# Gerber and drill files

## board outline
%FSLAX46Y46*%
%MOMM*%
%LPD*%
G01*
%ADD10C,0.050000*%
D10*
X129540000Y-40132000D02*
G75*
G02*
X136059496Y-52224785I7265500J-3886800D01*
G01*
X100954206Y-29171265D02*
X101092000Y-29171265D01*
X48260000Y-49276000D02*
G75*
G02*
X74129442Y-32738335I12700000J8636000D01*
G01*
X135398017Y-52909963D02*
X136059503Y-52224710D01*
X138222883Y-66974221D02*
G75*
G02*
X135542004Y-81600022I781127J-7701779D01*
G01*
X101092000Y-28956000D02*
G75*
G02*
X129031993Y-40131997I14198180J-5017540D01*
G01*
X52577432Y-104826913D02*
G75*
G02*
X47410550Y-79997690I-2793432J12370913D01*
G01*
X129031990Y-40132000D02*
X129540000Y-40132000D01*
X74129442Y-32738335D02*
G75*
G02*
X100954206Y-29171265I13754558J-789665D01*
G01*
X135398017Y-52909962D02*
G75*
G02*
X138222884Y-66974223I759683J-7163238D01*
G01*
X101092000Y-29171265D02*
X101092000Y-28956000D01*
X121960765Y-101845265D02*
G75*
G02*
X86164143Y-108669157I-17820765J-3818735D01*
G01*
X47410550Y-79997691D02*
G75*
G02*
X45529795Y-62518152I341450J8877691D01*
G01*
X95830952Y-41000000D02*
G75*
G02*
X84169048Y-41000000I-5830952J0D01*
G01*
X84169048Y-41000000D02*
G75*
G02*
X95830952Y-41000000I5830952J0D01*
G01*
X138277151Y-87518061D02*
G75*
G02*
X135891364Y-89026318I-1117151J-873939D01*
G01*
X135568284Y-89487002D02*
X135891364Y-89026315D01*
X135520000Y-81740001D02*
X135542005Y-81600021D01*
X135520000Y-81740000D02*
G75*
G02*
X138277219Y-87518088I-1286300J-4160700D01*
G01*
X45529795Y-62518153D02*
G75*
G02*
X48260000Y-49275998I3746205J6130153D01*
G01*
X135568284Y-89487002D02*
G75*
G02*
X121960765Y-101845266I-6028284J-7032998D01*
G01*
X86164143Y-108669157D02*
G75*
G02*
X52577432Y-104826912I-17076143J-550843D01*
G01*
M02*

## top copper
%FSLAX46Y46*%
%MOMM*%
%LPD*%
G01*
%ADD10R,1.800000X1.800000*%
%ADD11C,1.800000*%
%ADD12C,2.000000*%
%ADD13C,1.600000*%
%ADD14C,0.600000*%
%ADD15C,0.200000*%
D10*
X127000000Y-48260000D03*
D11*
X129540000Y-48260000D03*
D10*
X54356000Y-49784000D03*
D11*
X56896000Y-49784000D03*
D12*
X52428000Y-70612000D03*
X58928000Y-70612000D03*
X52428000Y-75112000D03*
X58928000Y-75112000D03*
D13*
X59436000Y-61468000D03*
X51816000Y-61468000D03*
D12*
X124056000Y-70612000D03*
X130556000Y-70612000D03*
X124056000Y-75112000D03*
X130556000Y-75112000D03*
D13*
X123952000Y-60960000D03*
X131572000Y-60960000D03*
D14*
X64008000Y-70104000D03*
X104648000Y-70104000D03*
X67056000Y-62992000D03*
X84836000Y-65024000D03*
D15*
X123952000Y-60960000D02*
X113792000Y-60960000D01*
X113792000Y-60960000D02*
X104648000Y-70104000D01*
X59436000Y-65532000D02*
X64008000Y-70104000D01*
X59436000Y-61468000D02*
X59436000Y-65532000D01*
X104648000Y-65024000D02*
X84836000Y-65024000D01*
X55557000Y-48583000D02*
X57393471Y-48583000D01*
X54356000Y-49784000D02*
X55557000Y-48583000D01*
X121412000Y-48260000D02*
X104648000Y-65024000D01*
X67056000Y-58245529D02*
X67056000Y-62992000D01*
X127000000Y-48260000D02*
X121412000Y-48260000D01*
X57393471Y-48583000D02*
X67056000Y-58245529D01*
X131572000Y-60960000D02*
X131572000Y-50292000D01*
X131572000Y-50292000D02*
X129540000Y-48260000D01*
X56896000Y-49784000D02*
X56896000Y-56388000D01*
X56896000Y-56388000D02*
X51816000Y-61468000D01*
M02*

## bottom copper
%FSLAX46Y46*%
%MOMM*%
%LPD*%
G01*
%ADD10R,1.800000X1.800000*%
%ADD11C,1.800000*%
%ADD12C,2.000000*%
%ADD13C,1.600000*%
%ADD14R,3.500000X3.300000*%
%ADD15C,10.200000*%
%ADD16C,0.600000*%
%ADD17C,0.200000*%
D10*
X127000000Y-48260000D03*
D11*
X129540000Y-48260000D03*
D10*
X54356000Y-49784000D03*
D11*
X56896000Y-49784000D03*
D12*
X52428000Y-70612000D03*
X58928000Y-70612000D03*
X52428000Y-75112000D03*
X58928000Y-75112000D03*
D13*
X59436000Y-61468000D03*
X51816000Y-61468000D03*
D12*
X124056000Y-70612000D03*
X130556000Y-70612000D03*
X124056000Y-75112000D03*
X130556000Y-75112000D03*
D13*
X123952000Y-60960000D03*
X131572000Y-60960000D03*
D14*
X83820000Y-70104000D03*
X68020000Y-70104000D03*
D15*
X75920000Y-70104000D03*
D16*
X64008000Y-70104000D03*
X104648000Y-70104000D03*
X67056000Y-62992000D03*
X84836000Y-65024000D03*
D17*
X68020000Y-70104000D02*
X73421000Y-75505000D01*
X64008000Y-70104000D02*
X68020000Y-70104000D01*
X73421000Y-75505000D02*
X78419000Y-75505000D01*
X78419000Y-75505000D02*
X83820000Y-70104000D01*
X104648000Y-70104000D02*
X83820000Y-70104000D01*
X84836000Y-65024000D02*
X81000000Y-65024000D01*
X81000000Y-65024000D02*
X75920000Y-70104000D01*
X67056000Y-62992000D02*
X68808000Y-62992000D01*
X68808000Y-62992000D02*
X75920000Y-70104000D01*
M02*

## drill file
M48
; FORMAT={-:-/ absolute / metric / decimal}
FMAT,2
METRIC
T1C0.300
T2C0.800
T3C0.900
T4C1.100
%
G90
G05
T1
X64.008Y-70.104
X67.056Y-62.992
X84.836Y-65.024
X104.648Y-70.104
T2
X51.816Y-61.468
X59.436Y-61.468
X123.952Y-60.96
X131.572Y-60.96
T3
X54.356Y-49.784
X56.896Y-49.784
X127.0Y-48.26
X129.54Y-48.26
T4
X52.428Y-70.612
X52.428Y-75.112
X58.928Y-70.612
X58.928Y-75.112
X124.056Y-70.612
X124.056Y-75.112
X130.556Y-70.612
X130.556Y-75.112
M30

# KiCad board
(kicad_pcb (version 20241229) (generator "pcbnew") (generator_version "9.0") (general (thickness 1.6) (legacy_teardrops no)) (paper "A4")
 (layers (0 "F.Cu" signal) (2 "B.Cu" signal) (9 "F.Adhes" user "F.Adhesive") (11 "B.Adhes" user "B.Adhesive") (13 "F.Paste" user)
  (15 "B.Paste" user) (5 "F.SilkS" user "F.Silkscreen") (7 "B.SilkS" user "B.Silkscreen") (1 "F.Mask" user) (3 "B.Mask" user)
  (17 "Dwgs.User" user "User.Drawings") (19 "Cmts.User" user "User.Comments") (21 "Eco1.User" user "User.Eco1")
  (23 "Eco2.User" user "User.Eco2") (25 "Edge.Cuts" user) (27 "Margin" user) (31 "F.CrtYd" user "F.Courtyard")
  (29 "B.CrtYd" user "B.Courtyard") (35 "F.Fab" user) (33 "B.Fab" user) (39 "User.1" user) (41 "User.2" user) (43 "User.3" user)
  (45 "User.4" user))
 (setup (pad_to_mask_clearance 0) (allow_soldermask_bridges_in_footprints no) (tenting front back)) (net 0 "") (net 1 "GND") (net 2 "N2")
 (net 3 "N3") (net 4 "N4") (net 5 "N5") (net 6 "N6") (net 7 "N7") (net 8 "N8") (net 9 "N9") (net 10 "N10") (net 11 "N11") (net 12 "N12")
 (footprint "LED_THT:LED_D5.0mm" (layer "F.Cu") (at 127 48.26)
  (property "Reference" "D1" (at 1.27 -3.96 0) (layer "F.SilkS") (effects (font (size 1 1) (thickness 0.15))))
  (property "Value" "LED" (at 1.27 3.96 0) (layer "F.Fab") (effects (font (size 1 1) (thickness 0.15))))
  (pad "1" thru_hole rect (at 0 0) (size 1.8 1.8) (drill 0.9) (layers "*.Cu" "*.Mask") (remove_unused_layers no) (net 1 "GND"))
  (pad "2" thru_hole circle (at 2.54 0) (size 1.8 1.8) (drill 0.9) (layers "*.Cu" "*.Mask") (remove_unused_layers no) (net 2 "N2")))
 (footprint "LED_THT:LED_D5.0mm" (layer "F.Cu") (at 54.356 49.784)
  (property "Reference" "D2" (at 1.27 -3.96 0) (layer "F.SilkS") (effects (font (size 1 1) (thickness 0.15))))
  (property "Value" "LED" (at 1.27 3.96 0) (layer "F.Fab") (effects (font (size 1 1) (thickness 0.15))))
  (pad "1" thru_hole rect (at 0 0) (size 1.8 1.8) (drill 0.9) (layers "*.Cu" "*.Mask") (remove_unused_layers no) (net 1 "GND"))
  (pad "2" thru_hole circle (at 2.54 0) (size 1.8 1.8) (drill 0.9) (layers "*.Cu" "*.Mask") (remove_unused_layers no) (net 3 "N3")))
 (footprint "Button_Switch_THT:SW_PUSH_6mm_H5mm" (layer "F.Cu") (at 52.428 70.612)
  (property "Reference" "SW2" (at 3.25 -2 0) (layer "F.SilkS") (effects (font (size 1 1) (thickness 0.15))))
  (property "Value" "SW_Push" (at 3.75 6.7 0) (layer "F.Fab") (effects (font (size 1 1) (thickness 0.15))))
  (pad "1" thru_hole circle (at 0 0 90) (size 2 2) (drill 1.1) (layers "*.Cu" "*.Mask") (remove_unused_layers no) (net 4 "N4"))
  (pad "1" thru_hole circle (at 6.5 0 90) (size 2 2) (drill 1.1) (layers "*.Cu" "*.Mask") (remove_unused_layers no) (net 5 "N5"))
  (pad "2" thru_hole circle (at 0 4.5 90) (size 2 2) (drill 1.1) (layers "*.Cu" "*.Mask") (remove_unused_layers no) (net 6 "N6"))
  (pad "2" thru_hole circle (at 6.5 4.5 90) (size 2 2) (drill 1.1) (layers "*.Cu" "*.Mask") (remove_unused_layers no) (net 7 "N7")))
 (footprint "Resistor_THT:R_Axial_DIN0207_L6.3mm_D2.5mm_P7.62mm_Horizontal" (layer "F.Cu") (at 59.436 61.468 180)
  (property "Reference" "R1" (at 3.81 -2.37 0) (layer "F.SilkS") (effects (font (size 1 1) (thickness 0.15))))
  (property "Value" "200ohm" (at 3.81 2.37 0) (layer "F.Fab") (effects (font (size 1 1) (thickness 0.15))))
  (pad "1" thru_hole circle (at 0 0 180) (size 1.6 1.6) (drill 0.8) (layers "*.Cu" "*.Mask") (remove_unused_layers no) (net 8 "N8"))
  (pad "2" thru_hole circle (at 7.62 0 180) (size 1.6 1.6) (drill 0.8) (layers "*.Cu" "*.Mask") (remove_unused_layers no) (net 3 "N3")))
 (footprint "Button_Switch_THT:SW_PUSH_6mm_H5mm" (layer "F.Cu") (at 124.056 70.612)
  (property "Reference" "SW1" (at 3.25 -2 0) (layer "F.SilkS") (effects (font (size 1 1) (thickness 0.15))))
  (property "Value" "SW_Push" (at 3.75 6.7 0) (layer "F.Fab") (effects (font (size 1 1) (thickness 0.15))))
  (pad "1" thru_hole circle (at 0 0 90) (size 2 2) (drill 1.1) (layers "*.Cu" "*.Mask") (remove_unused_layers no) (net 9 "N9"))
  (pad "1" thru_hole circle (at 6.5 0 90) (size 2 2) (drill 1.1) (layers "*.Cu" "*.Mask") (remove_unused_layers no) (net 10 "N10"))
  (pad "2" thru_hole circle (at 0 4.5 90) (size 2 2) (drill 1.1) (layers "*.Cu" "*.Mask") (remove_unused_layers no) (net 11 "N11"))
  (pad "2" thru_hole circle (at 6.5 4.5 90) (size 2 2) (drill 1.1) (layers "*.Cu" "*.Mask") (remove_unused_layers no) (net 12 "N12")))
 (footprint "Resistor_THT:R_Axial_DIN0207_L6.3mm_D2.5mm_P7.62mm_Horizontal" (layer "F.Cu") (at 123.952 60.96)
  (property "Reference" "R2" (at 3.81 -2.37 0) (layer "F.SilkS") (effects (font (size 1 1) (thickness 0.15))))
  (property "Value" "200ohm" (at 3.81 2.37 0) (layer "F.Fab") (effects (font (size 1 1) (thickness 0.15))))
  (pad "1" thru_hole circle (at 0 0) (size 1.6 1.6) (drill 0.8) (layers "*.Cu" "*.Mask") (remove_unused_layers no) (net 8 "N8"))
  (pad "2" thru_hole circle (at 7.62 0) (size 1.6 1.6) (drill 0.8) (layers "*.Cu" "*.Mask") (remove_unused_layers no) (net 2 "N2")))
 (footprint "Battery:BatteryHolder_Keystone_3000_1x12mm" (layer "B.Cu") (at 75.92 70.104 180)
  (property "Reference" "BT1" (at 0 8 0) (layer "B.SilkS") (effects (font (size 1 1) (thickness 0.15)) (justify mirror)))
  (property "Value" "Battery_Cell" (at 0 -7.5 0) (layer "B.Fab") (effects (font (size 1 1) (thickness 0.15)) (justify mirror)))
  (pad "1" smd rect (at -7.9 0 180) (size 3.5 3.3) (layers "B.Cu" "B.Mask" "B.Paste") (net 8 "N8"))
  (pad "1" smd rect (at 7.9 0 180) (size 3.5 3.3) (layers "B.Cu" "B.Mask" "B.Paste") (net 8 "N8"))
  (pad "2" smd circle (at 0 0 180) (size 10.2 10.2) (layers "B.Cu" "B.Mask") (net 1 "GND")))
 (gr_arc (start 129.54 40.132) (mid 144.058392 40.108523) (end 136.059503 52.224712) (stroke (width 0.05) (type default))
  (layer "Edge.Cuts"))
 (gr_line (start 100.954206 29.171265) (end 101.092 29.171265) (stroke (width 0.05) (type default)) (layer "Edge.Cuts"))
 (gr_arc (start 48.26 49.276) (mid 52.687837 27.700069) (end 74.129442 32.738335) (stroke (width 0.05) (type default)) (layer "Edge.Cuts"))
 (gr_line (start 135.398017 52.909963) (end 136.059503 52.22471) (stroke (width 0.05) (type default)) (layer "Edge.Cuts"))
 (gr_arc (start 138.222883 66.974221) (mid 146.618446 76.071709) (end 135.542005 81.60002) (stroke (width 0.05) (type default))
  (layer "Edge.Cuts"))
 (gr_arc (start 101.092 28.956) (mid 120.882838 19.991901) (end 129.032 40.132) (stroke (width 0.05) (type default)) (layer "Edge.Cuts"))
 (gr_arc (start 52.577432 104.826913) (mid 37.367613 95.039811) (end 47.41055 79.99769) (stroke (width 0.05) (type default))
  (layer "Edge.Cuts"))
 (gr_line (start 129.03199 40.132) (end 129.54 40.132) (stroke (width 0.05) (type default)) (layer "Edge.Cuts"))
 (gr_arc (start 74.129442 32.738335) (mid 86.067938 19.871011) (end 100.954206 29.171265) (stroke (width 0.05) (type default))
  (layer "Edge.Cuts"))
 (gr_arc (start 135.398017 52.909962) (mid 143.220055 58.654695) (end 138.222883 66.974221) (stroke (width 0.05) (type default))
  (layer "Edge.Cuts"))
 (gr_line (start 101.092 29.171265) (end 101.092 28.956) (stroke (width 0.05) (type default)) (layer "Edge.Cuts"))
 (gr_arc (start 121.960765 101.845265) (mid 107.552827 123.566933) (end 86.164143 108.669157) (stroke (width 0.05) (type default))
  (layer "Edge.Cuts"))
 (gr_arc (start 47.41055 79.997691) (mid 38.91873 72.070438) (end 45.529795 62.518152) (stroke (width 0.05) (type default))
  (layer "Edge.Cuts"))
 (gr_circle (center 90 41) (end 85 38) (stroke (width 0.05) (type default)) (fill no) (layer "Edge.Cuts"))
 (gr_arc (start 138.277151 87.518061) (mid 137.917923 89.590895) (end 135.891364 89.026318) (stroke (width 0.05) (type default))
  (layer "Edge.Cuts"))
 (gr_line (start 135.568284 89.487002) (end 135.891364 89.026315) (stroke (width 0.05) (type default)) (layer "Edge.Cuts"))
 (gr_line (start 135.52 81.740001) (end 135.542005 81.600021) (stroke (width 0.05) (type default)) (layer "Edge.Cuts"))
 (gr_arc (start 135.52 81.74) (mid 138.164098 84.025154) (end 138.277153 87.518061) (stroke (width 0.05) (type default)) (layer "Edge.Cuts"))
 (gr_arc (start 45.529795 62.518153) (mid 42.239785 54.937306) (end 48.26 49.275998) (stroke (width 0.05) (type default))
  (layer "Edge.Cuts"))
 (gr_arc (start 135.568284 89.487002) (mid 135.767603 103.37713) (end 121.960765 101.845266) (stroke (width 0.05) (type default))
  (layer "Edge.Cuts"))
 (gr_arc (start 86.164143 108.669157) (mid 67.146176 126.194316) (end 52.577432 104.826912) (stroke (width 0.05) (type default))
  (layer "Edge.Cuts"))
 (segment (start 123.952 60.96) (end 113.792 60.96) (width 0.2) (layer "F.Cu") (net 8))
 (segment (start 113.792 60.96) (end 104.648 70.104) (width 0.2) (layer "F.Cu") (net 8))
 (segment (start 59.436 65.532) (end 64.008 70.104) (width 0.2) (layer "F.Cu") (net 8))
 (segment (start 59.436 61.468) (end 59.436 65.532) (width 0.2) (layer "F.Cu") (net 8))
 (via (at 64.008 70.104) (size 0.6) (drill 0.3) (layers "F.Cu" "B.Cu") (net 8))
 (via (at 104.648 70.104) (size 0.6) (drill 0.3) (layers "F.Cu" "B.Cu") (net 8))
 (segment (start 68.02 70.104) (end 73.421 75.505) (width 0.2) (layer "B.Cu") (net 8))
 (segment (start 64.008 70.104) (end 68.02 70.104) (width 0.2) (layer "B.Cu") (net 8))
 (segment (start 73.421 75.505) (end 78.419 75.505) (width 0.2) (layer "B.Cu") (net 8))
 (segment (start 78.419 75.505) (end 83.82 70.104) (width 0.2) (layer "B.Cu") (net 8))
 (segment (start 104.648 70.104) (end 83.82 70.104) (width 0.2) (layer "B.Cu") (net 8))
 (segment (start 104.648 65.024) (end 84.836 65.024) (width 0.2) (layer "F.Cu") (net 1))
 (segment (start 55.557 48.583) (end 57.393471 48.583) (width 0.2) (layer "F.Cu") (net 1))
 (segment (start 54.356 49.784) (end 55.557 48.583) (width 0.2) (layer "F.Cu") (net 1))
 (segment (start 121.412 48.26) (end 104.648 65.024) (width 0.2) (layer "F.Cu") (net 1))
 (segment (start 67.056 58.245529) (end 67.056 62.992) (width 0.2) (layer "F.Cu") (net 1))
 (segment (start 127 48.26) (end 121.412 48.26) (width 0.2) (layer "F.Cu") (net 1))
 (segment (start 57.393471 48.583) (end 67.056 58.245529) (width 0.2) (layer "F.Cu") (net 1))
 (via (at 67.056 62.992) (size 0.6) (drill 0.3) (layers "F.Cu" "B.Cu") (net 1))
 (via (at 84.836 65.024) (size 0.6) (drill 0.3) (layers "F.Cu" "B.Cu") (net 1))
 (segment (start 84.836 65.024) (end 81 65.024) (width 0.2) (layer "B.Cu") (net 1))
 (segment (start 81 65.024) (end 75.92 70.104) (width 0.2) (layer "B.Cu") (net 1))
 (segment (start 67.056 62.992) (end 68.808 62.992) (width 0.2) (layer "B.Cu") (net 1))
 (segment (start 68.808 62.992) (end 75.92 70.104) (width 0.2) (layer "B.Cu") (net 1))
 (segment (start 131.572 60.96) (end 131.572 50.292) (width 0.2) (layer "F.Cu") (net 2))
 (segment (start 131.572 50.292) (end 129.54 48.26) (width 0.2) (layer "F.Cu") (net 2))
 (segment (start 56.896 49.784) (end 56.896 56.388) (width 0.2) (layer "F.Cu") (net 3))
 (segment (start 56.896 56.388) (end 51.816 61.468) (width 0.2) (layer "F.Cu") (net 3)))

